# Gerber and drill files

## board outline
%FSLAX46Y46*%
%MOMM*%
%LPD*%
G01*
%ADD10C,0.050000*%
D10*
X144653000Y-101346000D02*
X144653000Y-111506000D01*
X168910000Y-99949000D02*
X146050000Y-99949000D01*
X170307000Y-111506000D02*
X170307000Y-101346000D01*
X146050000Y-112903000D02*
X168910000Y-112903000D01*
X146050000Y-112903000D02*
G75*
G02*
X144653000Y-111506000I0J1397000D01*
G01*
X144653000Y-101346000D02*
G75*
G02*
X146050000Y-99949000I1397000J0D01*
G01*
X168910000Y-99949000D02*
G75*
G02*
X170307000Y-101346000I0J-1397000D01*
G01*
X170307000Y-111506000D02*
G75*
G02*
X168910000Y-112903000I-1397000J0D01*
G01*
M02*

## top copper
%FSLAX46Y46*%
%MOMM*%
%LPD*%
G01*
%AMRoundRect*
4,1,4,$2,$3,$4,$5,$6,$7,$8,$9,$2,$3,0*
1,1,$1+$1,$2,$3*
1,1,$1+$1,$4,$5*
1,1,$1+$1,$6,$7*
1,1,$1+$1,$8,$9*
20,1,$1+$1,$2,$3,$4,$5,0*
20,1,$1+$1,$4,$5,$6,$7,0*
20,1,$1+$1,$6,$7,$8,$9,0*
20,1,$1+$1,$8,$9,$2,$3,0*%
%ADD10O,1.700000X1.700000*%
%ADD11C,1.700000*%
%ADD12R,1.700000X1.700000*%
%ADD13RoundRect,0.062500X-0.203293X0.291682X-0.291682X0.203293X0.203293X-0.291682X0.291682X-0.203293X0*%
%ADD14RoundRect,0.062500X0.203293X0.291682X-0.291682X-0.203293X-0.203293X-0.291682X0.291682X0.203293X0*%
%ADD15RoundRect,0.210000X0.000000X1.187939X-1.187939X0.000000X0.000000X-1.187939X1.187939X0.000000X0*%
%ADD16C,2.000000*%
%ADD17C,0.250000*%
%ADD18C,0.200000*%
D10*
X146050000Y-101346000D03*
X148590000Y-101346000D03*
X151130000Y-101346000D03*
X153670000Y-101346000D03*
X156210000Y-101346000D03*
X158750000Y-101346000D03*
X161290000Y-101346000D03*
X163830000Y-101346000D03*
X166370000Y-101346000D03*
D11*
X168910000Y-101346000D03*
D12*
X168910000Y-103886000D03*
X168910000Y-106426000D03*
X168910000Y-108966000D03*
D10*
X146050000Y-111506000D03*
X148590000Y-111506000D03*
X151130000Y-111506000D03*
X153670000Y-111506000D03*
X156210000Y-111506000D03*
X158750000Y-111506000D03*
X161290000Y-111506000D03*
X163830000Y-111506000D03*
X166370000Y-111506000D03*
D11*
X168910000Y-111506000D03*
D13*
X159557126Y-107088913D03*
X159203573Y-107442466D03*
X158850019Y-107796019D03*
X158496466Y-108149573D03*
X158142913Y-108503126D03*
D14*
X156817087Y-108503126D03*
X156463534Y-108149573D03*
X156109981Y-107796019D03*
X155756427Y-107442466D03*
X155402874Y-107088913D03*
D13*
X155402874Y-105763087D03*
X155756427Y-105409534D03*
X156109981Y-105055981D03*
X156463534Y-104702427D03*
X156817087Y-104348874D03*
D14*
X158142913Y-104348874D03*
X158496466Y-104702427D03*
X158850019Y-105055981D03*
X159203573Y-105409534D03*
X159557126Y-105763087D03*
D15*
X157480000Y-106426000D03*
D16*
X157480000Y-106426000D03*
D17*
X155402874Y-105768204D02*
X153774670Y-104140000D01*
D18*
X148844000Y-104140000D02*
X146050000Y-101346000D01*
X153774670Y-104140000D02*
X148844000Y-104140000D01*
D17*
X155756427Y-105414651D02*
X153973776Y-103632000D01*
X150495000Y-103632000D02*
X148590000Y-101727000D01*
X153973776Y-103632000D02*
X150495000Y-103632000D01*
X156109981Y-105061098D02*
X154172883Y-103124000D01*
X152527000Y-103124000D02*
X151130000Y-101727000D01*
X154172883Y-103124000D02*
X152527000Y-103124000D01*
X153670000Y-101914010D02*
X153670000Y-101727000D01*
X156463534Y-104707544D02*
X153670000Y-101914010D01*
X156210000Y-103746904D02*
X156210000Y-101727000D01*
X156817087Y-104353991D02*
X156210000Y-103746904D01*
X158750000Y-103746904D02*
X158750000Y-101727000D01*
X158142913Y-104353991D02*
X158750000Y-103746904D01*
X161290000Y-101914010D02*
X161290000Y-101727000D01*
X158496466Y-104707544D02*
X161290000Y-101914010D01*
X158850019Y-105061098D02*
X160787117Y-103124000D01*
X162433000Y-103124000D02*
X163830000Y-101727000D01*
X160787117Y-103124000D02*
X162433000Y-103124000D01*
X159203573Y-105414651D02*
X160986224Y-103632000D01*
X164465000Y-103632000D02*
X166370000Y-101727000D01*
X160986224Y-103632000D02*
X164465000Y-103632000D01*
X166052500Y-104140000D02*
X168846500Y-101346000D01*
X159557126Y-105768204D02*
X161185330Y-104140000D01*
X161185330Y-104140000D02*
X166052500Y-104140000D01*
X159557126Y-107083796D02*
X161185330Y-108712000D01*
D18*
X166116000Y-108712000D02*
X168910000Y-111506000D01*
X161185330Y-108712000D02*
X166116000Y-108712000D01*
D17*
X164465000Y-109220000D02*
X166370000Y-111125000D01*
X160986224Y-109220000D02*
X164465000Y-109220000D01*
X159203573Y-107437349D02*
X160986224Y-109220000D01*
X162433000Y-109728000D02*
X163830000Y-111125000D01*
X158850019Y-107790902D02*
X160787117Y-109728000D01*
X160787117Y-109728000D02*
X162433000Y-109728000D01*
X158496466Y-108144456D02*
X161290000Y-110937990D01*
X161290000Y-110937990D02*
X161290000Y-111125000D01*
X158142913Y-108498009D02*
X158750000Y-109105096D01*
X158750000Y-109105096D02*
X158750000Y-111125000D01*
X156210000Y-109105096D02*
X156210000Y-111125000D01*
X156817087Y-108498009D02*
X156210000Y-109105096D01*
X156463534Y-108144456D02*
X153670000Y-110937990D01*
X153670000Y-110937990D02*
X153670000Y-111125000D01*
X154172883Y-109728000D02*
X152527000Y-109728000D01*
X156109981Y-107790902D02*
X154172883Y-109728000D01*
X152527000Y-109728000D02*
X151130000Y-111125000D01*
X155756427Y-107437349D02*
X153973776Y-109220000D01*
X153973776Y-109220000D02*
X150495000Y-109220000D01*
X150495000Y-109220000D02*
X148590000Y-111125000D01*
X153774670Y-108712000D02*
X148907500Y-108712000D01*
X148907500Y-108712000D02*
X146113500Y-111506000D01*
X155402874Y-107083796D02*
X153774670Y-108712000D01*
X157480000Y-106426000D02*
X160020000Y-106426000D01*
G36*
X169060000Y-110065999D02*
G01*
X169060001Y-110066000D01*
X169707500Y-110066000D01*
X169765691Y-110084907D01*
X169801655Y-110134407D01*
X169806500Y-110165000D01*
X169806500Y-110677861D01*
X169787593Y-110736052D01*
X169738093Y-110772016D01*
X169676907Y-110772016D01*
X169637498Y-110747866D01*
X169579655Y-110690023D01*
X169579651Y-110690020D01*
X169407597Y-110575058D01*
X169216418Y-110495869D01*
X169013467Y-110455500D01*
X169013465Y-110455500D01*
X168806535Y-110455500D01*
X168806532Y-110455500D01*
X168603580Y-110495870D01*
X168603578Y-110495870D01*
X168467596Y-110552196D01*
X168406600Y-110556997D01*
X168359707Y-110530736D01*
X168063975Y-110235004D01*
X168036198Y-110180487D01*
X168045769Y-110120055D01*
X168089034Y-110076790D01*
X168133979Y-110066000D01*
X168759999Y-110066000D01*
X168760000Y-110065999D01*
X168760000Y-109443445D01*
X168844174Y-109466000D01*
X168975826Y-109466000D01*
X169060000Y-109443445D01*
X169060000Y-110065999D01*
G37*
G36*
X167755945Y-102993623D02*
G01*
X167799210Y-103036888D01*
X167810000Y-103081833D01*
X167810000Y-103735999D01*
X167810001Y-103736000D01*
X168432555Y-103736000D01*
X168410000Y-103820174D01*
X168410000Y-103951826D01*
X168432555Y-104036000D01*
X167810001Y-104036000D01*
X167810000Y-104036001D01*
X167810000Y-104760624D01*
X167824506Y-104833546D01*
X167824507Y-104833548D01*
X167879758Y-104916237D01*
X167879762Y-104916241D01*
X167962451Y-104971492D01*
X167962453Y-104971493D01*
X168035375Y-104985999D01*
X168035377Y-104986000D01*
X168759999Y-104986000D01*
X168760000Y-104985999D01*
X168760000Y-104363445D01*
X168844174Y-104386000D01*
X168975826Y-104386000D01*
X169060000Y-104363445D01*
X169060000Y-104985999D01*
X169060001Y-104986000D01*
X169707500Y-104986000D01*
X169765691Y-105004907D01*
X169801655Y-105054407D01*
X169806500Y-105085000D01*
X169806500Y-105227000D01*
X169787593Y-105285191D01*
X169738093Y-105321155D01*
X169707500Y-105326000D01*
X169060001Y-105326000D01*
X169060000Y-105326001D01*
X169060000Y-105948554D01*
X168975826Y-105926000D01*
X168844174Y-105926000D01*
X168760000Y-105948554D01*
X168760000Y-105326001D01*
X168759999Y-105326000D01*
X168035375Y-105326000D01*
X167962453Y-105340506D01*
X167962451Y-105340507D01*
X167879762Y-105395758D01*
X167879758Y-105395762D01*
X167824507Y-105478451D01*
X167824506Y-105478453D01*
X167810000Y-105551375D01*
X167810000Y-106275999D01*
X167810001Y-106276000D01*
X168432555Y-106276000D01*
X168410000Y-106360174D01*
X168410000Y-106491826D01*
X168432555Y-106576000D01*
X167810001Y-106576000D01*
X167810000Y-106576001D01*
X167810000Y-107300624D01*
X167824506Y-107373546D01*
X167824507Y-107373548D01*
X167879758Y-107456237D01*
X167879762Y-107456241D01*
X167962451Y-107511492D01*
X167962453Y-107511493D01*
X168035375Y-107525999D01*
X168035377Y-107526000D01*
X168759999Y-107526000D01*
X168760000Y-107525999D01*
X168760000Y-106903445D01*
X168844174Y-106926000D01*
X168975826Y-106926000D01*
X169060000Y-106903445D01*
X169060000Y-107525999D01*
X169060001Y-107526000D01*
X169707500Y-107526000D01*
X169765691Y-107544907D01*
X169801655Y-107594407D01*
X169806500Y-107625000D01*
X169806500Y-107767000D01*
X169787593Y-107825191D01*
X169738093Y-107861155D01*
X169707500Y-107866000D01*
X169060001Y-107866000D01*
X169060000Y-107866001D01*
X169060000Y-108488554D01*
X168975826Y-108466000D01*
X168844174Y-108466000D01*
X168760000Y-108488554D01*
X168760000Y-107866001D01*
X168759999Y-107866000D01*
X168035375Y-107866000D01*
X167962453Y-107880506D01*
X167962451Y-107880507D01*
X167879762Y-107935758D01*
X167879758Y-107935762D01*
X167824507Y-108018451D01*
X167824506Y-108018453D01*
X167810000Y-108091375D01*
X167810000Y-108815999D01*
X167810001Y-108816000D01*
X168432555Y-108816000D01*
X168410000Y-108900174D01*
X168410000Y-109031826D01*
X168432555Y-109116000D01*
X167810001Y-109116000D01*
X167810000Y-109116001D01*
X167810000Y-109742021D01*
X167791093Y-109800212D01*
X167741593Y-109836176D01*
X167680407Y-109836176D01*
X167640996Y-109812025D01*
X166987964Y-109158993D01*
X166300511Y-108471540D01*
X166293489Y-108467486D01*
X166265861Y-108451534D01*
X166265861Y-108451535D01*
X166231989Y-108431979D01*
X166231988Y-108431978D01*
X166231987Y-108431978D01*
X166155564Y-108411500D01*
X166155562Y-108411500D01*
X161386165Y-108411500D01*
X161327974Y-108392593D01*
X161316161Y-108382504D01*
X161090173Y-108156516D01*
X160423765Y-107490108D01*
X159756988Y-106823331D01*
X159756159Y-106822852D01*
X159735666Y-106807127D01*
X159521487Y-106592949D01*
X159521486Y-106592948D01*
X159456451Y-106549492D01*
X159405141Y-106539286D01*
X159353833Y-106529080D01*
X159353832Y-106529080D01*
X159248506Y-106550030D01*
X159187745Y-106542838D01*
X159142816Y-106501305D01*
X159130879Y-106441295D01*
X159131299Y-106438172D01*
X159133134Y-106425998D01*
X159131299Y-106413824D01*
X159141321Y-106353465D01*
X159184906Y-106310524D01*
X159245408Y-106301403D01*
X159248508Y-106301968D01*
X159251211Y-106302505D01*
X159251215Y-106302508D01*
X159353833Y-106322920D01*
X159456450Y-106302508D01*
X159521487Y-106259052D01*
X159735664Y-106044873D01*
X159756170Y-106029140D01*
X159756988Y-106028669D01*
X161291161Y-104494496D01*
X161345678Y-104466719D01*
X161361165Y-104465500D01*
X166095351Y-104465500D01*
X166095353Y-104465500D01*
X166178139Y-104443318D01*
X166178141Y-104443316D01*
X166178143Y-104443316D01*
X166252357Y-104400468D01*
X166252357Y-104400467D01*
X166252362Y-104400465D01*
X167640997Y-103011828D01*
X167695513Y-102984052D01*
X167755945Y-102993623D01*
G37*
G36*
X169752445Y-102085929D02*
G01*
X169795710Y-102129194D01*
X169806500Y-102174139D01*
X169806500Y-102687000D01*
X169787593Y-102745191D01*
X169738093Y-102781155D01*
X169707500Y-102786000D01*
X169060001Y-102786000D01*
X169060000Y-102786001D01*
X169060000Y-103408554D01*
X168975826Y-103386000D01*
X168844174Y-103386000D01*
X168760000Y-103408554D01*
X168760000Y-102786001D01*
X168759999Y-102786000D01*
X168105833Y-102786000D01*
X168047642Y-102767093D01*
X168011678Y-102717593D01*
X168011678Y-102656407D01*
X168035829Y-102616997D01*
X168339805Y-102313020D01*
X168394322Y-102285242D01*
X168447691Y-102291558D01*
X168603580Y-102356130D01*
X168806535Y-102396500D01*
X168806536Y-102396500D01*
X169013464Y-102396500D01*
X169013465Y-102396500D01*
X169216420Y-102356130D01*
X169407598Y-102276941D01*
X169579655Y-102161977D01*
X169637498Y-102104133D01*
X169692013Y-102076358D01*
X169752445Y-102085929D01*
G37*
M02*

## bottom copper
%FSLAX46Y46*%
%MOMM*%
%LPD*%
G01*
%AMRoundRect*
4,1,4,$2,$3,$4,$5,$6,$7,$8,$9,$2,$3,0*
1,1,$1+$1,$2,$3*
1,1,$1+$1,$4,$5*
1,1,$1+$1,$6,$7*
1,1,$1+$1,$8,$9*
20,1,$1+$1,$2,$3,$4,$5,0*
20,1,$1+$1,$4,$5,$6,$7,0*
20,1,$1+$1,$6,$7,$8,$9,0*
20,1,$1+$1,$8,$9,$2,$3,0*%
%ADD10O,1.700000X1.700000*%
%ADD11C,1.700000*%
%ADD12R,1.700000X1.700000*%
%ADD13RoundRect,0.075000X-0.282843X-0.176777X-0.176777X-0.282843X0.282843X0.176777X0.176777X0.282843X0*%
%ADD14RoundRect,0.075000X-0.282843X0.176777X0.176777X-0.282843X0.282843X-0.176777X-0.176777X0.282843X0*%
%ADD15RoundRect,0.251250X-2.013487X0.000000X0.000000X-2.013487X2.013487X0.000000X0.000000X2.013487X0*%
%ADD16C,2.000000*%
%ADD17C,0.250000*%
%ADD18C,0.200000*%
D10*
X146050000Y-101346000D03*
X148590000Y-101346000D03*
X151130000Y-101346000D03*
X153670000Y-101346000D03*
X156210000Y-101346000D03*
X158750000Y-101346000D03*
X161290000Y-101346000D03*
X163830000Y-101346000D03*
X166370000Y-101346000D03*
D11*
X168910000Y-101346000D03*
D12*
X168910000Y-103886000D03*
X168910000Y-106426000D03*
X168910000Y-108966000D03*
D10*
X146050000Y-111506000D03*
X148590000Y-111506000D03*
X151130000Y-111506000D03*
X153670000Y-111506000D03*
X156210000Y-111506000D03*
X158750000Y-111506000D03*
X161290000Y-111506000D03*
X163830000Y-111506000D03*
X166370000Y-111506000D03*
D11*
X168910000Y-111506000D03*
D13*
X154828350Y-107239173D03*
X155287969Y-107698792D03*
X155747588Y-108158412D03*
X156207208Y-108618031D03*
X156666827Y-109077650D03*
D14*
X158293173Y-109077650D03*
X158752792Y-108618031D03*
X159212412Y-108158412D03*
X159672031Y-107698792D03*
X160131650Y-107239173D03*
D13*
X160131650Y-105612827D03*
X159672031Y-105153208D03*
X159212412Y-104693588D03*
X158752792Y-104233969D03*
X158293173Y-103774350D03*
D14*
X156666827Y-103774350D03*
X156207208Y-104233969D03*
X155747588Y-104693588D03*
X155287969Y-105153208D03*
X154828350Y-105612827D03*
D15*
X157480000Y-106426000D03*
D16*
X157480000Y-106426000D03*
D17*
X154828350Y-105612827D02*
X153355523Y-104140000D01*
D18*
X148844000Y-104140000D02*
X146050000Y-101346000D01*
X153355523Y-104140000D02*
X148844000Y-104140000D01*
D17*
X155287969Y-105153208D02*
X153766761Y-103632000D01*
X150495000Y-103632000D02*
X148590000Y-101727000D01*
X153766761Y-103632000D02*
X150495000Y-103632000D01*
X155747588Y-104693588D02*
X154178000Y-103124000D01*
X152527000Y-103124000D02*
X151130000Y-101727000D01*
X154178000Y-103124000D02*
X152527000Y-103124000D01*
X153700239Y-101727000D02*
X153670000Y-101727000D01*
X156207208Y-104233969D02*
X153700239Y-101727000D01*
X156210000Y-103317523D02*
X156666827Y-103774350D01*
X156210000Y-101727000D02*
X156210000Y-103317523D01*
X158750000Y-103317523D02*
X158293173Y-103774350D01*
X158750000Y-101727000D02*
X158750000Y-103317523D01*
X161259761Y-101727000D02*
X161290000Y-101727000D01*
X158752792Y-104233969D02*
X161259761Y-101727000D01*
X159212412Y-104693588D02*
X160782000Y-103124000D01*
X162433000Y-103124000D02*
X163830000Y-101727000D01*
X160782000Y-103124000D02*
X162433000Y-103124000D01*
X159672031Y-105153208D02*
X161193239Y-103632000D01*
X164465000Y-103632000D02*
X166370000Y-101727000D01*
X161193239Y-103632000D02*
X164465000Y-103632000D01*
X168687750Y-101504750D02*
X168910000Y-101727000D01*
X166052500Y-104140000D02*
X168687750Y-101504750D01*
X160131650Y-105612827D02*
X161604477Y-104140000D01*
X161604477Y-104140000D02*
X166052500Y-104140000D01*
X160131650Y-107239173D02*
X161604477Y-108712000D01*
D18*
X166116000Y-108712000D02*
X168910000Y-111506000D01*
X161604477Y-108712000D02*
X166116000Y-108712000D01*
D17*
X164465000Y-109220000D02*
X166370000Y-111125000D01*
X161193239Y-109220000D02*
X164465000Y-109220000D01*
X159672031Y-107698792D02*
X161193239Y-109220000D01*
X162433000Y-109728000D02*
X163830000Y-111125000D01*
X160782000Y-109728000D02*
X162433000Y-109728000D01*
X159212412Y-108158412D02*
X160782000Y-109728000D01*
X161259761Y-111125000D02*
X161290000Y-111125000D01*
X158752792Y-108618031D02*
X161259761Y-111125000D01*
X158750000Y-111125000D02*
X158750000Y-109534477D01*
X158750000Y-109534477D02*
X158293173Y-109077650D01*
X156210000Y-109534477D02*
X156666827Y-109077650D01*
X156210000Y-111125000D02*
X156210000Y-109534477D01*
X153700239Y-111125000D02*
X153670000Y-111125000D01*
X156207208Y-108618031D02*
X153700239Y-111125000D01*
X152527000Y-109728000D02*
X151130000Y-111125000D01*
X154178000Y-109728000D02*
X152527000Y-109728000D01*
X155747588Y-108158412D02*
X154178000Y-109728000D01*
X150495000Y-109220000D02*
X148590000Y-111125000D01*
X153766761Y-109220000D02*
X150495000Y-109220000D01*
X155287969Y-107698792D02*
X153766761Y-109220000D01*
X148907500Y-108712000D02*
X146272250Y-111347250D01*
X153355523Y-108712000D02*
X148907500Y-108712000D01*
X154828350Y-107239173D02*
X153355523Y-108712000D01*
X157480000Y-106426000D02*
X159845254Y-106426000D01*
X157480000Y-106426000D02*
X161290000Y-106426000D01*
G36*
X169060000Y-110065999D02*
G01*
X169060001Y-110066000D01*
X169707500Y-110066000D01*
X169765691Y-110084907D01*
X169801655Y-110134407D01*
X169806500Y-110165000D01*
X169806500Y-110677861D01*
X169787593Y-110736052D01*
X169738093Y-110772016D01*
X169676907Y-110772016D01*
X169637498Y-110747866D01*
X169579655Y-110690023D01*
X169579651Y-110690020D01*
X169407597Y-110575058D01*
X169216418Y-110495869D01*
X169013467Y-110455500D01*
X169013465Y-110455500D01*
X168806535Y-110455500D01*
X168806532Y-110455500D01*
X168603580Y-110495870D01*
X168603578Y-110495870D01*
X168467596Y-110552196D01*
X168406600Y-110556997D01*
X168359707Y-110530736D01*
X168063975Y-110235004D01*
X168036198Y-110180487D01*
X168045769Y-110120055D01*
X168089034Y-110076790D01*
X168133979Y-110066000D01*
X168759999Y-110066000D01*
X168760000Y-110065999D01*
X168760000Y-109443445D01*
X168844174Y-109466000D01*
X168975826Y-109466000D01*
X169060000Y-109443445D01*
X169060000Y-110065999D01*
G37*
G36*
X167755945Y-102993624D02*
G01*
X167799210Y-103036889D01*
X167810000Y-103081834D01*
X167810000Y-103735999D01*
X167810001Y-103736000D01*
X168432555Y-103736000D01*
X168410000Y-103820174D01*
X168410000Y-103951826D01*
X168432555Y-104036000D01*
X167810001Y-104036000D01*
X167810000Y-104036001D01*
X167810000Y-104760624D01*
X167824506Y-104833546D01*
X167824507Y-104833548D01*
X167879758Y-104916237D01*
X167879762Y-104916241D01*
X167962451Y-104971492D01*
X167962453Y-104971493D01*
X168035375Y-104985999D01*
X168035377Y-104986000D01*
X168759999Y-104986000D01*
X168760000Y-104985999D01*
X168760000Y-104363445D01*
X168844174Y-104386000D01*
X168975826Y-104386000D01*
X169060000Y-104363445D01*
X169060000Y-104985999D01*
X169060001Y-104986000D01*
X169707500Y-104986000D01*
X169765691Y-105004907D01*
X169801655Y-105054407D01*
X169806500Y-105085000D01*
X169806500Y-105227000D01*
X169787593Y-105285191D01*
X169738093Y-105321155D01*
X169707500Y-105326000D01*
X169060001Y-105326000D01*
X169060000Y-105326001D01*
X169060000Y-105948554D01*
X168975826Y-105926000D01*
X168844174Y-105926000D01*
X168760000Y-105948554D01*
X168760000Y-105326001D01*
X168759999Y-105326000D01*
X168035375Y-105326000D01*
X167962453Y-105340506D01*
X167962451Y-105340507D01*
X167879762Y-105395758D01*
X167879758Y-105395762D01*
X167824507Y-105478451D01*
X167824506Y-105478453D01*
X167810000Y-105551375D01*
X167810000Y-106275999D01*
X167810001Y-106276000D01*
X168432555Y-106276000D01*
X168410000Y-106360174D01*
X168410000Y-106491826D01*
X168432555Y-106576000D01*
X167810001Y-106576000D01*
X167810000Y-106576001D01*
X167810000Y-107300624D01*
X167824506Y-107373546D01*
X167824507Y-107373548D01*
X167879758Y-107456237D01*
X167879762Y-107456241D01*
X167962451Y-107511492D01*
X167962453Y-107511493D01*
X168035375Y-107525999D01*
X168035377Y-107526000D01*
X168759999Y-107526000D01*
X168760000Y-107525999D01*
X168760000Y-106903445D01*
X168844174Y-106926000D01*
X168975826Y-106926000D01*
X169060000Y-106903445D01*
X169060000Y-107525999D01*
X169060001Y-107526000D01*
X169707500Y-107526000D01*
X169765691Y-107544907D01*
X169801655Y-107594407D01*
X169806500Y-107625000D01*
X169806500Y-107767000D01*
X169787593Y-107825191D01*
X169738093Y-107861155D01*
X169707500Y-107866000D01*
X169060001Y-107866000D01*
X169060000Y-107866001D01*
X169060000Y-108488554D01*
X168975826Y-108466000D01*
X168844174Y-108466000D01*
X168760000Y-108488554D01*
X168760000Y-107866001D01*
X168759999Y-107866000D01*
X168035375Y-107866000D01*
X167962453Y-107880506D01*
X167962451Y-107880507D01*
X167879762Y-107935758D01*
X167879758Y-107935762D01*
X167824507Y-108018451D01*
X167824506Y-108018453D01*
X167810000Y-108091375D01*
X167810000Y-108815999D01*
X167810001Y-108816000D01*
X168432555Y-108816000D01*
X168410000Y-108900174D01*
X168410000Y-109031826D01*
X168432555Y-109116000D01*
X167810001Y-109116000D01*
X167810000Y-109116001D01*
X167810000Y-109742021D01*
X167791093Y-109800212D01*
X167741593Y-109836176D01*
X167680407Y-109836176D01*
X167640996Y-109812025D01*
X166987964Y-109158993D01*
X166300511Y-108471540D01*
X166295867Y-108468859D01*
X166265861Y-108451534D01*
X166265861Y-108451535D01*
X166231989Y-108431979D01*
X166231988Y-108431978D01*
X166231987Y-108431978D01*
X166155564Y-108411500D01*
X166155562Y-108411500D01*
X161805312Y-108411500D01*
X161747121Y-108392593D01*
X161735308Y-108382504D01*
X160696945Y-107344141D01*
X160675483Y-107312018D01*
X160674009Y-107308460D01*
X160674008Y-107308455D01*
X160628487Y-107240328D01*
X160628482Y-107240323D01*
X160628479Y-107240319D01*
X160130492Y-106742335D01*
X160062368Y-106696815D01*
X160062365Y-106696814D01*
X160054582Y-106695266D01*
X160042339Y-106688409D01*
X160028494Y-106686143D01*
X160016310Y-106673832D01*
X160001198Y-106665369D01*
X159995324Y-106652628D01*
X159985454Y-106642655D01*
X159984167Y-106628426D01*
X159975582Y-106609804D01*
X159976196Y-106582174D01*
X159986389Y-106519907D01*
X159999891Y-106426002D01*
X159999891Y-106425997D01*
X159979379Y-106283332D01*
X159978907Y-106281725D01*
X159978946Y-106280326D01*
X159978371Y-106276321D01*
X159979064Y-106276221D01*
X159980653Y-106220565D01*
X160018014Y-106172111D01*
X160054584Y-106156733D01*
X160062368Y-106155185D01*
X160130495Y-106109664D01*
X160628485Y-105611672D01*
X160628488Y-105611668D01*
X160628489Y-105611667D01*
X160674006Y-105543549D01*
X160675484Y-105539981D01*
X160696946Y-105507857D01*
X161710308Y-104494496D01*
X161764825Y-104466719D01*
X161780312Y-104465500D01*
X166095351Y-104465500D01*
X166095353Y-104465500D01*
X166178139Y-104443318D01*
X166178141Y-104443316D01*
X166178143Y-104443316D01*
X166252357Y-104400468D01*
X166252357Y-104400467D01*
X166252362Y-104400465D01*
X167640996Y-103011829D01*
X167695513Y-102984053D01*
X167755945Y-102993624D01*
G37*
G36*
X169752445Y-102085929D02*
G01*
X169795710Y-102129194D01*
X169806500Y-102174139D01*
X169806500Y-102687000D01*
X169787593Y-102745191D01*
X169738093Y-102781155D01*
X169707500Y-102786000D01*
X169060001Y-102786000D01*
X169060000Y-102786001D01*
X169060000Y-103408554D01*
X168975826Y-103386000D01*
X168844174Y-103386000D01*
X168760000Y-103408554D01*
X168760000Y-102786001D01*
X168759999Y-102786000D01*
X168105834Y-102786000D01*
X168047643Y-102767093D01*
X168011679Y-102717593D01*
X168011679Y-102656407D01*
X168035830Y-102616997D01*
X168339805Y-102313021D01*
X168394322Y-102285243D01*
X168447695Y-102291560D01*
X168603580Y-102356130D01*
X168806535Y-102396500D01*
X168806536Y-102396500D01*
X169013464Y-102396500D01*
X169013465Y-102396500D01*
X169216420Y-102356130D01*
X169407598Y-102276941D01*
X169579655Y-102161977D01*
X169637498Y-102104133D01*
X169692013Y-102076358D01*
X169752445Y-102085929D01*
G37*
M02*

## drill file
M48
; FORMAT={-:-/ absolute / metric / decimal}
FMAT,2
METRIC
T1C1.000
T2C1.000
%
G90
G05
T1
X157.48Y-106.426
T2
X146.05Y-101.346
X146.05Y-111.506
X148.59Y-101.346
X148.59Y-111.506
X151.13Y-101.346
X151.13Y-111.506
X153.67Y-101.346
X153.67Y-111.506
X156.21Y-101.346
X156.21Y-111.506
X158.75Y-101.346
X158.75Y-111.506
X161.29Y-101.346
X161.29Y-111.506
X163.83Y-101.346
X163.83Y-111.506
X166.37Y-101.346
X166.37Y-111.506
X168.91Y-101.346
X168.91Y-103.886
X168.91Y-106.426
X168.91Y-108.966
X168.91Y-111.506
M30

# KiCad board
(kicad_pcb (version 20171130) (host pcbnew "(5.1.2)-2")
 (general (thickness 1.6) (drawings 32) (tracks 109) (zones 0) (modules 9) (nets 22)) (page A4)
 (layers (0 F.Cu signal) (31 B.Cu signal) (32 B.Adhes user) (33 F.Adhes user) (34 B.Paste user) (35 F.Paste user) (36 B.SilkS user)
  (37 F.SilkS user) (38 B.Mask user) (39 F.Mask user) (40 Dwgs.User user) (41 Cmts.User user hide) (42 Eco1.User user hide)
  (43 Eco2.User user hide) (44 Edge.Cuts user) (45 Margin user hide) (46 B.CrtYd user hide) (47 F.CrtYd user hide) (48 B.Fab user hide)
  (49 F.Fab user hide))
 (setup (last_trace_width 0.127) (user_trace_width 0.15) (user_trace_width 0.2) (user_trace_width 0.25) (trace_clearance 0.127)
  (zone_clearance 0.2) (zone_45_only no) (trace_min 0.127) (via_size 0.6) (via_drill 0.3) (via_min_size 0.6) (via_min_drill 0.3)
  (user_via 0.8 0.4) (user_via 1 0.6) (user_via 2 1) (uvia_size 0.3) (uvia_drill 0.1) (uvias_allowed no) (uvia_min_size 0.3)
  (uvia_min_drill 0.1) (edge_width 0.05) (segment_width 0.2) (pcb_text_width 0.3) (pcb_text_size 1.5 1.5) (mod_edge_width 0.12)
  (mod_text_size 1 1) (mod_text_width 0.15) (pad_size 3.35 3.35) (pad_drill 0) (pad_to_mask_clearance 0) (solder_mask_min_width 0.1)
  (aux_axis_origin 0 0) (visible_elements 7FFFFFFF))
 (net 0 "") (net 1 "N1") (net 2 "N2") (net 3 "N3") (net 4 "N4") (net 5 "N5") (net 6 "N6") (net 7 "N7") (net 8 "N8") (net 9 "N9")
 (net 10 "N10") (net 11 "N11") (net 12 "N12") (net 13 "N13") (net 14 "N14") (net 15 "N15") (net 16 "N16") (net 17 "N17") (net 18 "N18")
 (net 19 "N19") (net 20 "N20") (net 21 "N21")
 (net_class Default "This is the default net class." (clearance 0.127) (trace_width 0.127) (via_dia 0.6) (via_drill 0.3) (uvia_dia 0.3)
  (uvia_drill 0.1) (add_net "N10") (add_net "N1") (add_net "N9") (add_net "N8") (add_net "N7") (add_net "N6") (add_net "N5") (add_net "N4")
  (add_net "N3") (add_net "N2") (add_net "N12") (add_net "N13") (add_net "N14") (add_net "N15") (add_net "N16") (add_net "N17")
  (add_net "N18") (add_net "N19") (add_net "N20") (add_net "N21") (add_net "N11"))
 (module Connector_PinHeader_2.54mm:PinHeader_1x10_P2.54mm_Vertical (layer F.Cu) (at 168.91 101.346 270)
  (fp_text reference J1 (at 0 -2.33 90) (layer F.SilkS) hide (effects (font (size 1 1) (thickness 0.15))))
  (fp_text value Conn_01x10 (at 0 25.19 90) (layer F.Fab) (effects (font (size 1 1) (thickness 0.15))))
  (pad 10 thru_hole oval (at 0 22.86 270) (size 1.7 1.7) (drill 1) (layers *.Cu *.Mask) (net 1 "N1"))
  (pad 9 thru_hole oval (at 0 20.32 270) (size 1.7 1.7) (drill 1) (layers *.Cu *.Mask) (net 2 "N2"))
  (pad 8 thru_hole oval (at 0 17.78 270) (size 1.7 1.7) (drill 1) (layers *.Cu *.Mask) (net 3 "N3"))
  (pad 7 thru_hole oval (at 0 15.24 270) (size 1.7 1.7) (drill 1) (layers *.Cu *.Mask) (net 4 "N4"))
  (pad 6 thru_hole oval (at 0 12.7 270) (size 1.7 1.7) (drill 1) (layers *.Cu *.Mask) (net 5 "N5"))
  (pad 5 thru_hole oval (at 0 10.16 270) (size 1.7 1.7) (drill 1) (layers *.Cu *.Mask) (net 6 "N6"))
  (pad 4 thru_hole oval (at 0 7.62 270) (size 1.7 1.7) (drill 1) (layers *.Cu *.Mask) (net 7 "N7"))
  (pad 3 thru_hole oval (at 0 5.08 270) (size 1.7 1.7) (drill 1) (layers *.Cu *.Mask) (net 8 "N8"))
  (pad 2 thru_hole oval (at 0 2.54 270) (size 1.7 1.7) (drill 1) (layers *.Cu *.Mask) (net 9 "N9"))
  (pad 1 thru_hole circle (at 0 0 270) (size 1.7 1.7) (drill 1) (layers *.Cu *.Mask) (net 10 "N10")))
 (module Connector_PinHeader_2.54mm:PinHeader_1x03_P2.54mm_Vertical (layer B.Cu) (at 168.91 103.886 180)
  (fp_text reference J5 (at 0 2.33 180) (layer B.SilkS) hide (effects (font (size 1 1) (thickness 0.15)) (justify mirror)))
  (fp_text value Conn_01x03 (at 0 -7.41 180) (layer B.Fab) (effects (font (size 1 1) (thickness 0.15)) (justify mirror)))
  (pad 1 thru_hole rect (at 0 0 180) (size 1.7 1.7) (drill 1) (layers *.Cu *.Mask) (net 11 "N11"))
  (pad 2 thru_hole rect (at 0 -2.54 180) (size 1.7 1.7) (drill 1) (layers *.Cu *.Mask) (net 11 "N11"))
  (pad 3 thru_hole rect (at 0 -5.08 180) (size 1.7 1.7) (drill 1) (layers *.Cu *.Mask) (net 11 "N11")))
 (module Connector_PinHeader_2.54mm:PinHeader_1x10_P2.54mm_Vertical (layer F.Cu) (at 168.91 111.506 270)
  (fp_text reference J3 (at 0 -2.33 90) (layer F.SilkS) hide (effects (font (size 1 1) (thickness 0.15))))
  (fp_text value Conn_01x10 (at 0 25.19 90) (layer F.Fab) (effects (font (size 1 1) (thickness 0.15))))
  (pad 10 thru_hole oval (at 0 22.86 270) (size 1.7 1.7) (drill 1) (layers *.Cu *.Mask) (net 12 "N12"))
  (pad 9 thru_hole oval (at 0 20.32 270) (size 1.7 1.7) (drill 1) (layers *.Cu *.Mask) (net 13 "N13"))
  (pad 8 thru_hole oval (at 0 17.78 270) (size 1.7 1.7) (drill 1) (layers *.Cu *.Mask) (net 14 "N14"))
  (pad 7 thru_hole oval (at 0 15.24 270) (size 1.7 1.7) (drill 1) (layers *.Cu *.Mask) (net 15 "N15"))
  (pad 6 thru_hole oval (at 0 12.7 270) (size 1.7 1.7) (drill 1) (layers *.Cu *.Mask) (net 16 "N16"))
  (pad 5 thru_hole oval (at 0 10.16 270) (size 1.7 1.7) (drill 1) (layers *.Cu *.Mask) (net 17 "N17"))
  (pad 4 thru_hole oval (at 0 7.62 270) (size 1.7 1.7) (drill 1) (layers *.Cu *.Mask) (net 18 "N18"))
  (pad 3 thru_hole oval (at 0 5.08 270) (size 1.7 1.7) (drill 1) (layers *.Cu *.Mask) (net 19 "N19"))
  (pad 2 thru_hole oval (at 0 2.54 270) (size 1.7 1.7) (drill 1) (layers *.Cu *.Mask) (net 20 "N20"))
  (pad 1 thru_hole circle (at 0 0 270) (size 1.7 1.7) (drill 1) (layers *.Cu *.Mask) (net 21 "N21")))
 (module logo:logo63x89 (layer B.Cu) (at 148.209 106.299 270)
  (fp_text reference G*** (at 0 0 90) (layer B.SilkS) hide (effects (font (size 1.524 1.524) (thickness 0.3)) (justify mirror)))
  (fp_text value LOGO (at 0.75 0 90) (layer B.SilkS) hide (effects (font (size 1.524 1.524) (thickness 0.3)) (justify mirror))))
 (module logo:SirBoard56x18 (layer B.Cu) (at 152.654 106.426 270)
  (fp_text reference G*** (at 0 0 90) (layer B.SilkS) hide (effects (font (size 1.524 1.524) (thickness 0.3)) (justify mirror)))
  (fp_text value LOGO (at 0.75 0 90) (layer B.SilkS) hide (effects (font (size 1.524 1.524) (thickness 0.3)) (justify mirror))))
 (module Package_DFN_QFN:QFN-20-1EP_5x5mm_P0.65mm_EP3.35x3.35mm (layer B.Cu) (at 157.48 106.426 315)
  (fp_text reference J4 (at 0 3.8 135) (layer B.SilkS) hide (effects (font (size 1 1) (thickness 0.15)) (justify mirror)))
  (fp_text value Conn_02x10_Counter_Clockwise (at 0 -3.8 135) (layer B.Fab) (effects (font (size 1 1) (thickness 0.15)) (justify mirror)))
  (pad 20 smd roundrect (at -1.3 2.45 315) (size 0.3 0.8) (layers B.Cu B.Paste B.Mask) (roundrect_rratio 0.25) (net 12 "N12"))
  (pad 19 smd roundrect (at -0.65 2.45 315) (size 0.3 0.8) (layers B.Cu B.Paste B.Mask) (roundrect_rratio 0.25) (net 13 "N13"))
  (pad 18 smd roundrect (at 0 2.45 315) (size 0.3 0.8) (layers B.Cu B.Paste B.Mask) (roundrect_rratio 0.25) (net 14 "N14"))
  (pad 17 smd roundrect (at 0.65 2.45 315) (size 0.3 0.8) (layers B.Cu B.Paste B.Mask) (roundrect_rratio 0.25) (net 15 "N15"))
  (pad 16 smd roundrect (at 1.3 2.45 315) (size 0.3 0.8) (layers B.Cu B.Paste B.Mask) (roundrect_rratio 0.25) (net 16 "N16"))
  (pad 15 smd roundrect (at 2.45 1.3 315) (size 0.8 0.3) (layers B.Cu B.Paste B.Mask) (roundrect_rratio 0.25) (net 17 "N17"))
  (pad 14 smd roundrect (at 2.45 0.65 315) (size 0.8 0.3) (layers B.Cu B.Paste B.Mask) (roundrect_rratio 0.25) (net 18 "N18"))
  (pad 13 smd roundrect (at 2.45 0 315) (size 0.8 0.3) (layers B.Cu B.Paste B.Mask) (roundrect_rratio 0.25) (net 19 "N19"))
  (pad 12 smd roundrect (at 2.45 -0.65 315) (size 0.8 0.3) (layers B.Cu B.Paste B.Mask) (roundrect_rratio 0.25) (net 20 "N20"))
  (pad 11 smd roundrect (at 2.45 -1.3 315) (size 0.8 0.3) (layers B.Cu B.Paste B.Mask) (roundrect_rratio 0.25) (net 21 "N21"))
  (pad 10 smd roundrect (at 1.3 -2.45 315) (size 0.3 0.8) (layers B.Cu B.Paste B.Mask) (roundrect_rratio 0.25) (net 10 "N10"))
  (pad 9 smd roundrect (at 0.65 -2.45 315) (size 0.3 0.8) (layers B.Cu B.Paste B.Mask) (roundrect_rratio 0.25) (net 9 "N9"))
  (pad 8 smd roundrect (at 0 -2.45 315) (size 0.3 0.8) (layers B.Cu B.Paste B.Mask) (roundrect_rratio 0.25) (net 8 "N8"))
  (pad 7 smd roundrect (at -0.65 -2.45 315) (size 0.3 0.8) (layers B.Cu B.Paste B.Mask) (roundrect_rratio 0.25) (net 7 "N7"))
  (pad 6 smd roundrect (at -1.3 -2.45 315) (size 0.3 0.8) (layers B.Cu B.Paste B.Mask) (roundrect_rratio 0.25) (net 6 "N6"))
  (pad 5 smd roundrect (at -2.45 -1.3 315) (size 0.8 0.3) (layers B.Cu B.Paste B.Mask) (roundrect_rratio 0.25) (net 5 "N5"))
  (pad 4 smd roundrect (at -2.45 -0.65 315) (size 0.8 0.3) (layers B.Cu B.Paste B.Mask) (roundrect_rratio 0.25) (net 4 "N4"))
  (pad 3 smd roundrect (at -2.45 0 315) (size 0.8 0.3) (layers B.Cu B.Paste B.Mask) (roundrect_rratio 0.25) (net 3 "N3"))
  (pad 2 smd roundrect (at -2.45 0.65 315) (size 0.8 0.3) (layers B.Cu B.Paste B.Mask) (roundrect_rratio 0.25) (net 2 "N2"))
  (pad 1 smd roundrect (at -2.45 1.3 315) (size 0.8 0.3) (layers B.Cu B.Paste B.Mask) (roundrect_rratio 0.25) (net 1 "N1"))
  (pad "" smd roundrect (at 0.84 -0.84 315) (size 1.35 1.35) (layers B.Paste) (roundrect_rratio 0.185185))
  (pad "" smd roundrect (at 0.84 0.84 315) (size 1.35 1.35) (layers B.Paste) (roundrect_rratio 0.185185))
  (pad "" smd roundrect (at -0.84 -0.84 315) (size 1.35 1.35) (layers B.Paste) (roundrect_rratio 0.185185))
  (pad "" smd roundrect (at -0.84 0.84 315) (size 1.35 1.35) (layers B.Paste) (roundrect_rratio 0.185185))
  (pad 21 smd roundrect (at 0 0 315) (size 3.35 3.35) (layers B.Cu B.Mask) (roundrect_rratio 0.075) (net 11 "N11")))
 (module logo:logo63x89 (layer F.Cu) (at 148.336 106.426 90)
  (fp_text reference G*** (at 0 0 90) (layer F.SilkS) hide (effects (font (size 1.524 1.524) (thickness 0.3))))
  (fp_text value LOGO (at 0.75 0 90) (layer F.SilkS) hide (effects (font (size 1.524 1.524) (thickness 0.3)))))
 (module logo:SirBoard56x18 (layer F.Cu) (at 152.654 106.426 90)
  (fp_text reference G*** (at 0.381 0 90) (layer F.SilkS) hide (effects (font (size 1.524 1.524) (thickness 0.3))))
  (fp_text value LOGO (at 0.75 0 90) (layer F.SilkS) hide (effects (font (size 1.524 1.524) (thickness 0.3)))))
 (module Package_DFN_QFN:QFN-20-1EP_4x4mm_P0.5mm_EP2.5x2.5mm (layer F.Cu) (at 157.48 106.426 225)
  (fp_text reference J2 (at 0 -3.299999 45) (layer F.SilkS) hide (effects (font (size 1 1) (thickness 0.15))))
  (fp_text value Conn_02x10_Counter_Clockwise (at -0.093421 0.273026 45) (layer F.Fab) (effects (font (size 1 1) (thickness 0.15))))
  (pad 20 smd roundrect (at -1 -1.9375 225) (size 0.25 0.825) (layers F.Cu F.Paste F.Mask) (roundrect_rratio 0.25) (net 21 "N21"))
  (pad 19 smd roundrect (at -0.5 -1.9375 225) (size 0.25 0.825) (layers F.Cu F.Paste F.Mask) (roundrect_rratio 0.25) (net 20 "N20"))
  (pad 18 smd roundrect (at 0 -1.9375 225) (size 0.25 0.825) (layers F.Cu F.Paste F.Mask) (roundrect_rratio 0.25) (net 19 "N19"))
  (pad 17 smd roundrect (at 0.5 -1.9375 225) (size 0.25 0.825) (layers F.Cu F.Paste F.Mask) (roundrect_rratio 0.25) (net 18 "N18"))
  (pad 16 smd roundrect (at 1 -1.9375 225) (size 0.25 0.825) (layers F.Cu F.Paste F.Mask) (roundrect_rratio 0.25) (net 17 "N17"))
  (pad 15 smd roundrect (at 1.9375 -1 225) (size 0.825 0.25) (layers F.Cu F.Paste F.Mask) (roundrect_rratio 0.25) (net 16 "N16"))
  (pad 14 smd roundrect (at 1.9375 -0.5 225) (size 0.825 0.25) (layers F.Cu F.Paste F.Mask) (roundrect_rratio 0.25) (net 15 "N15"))
  (pad 13 smd roundrect (at 1.9375 0 225) (size 0.825 0.25) (layers F.Cu F.Paste F.Mask) (roundrect_rratio 0.25) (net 14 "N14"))
  (pad 12 smd roundrect (at 1.9375 0.5 225) (size 0.825 0.25) (layers F.Cu F.Paste F.Mask) (roundrect_rratio 0.25) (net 13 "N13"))
  (pad 11 smd roundrect (at 1.9375 1 225) (size 0.825 0.25) (layers F.Cu F.Paste F.Mask) (roundrect_rratio 0.25) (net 12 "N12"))
  (pad 10 smd roundrect (at 1 1.9375 225) (size 0.25 0.825) (layers F.Cu F.Paste F.Mask) (roundrect_rratio 0.25) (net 1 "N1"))
  (pad 9 smd roundrect (at 0.5 1.9375 225) (size 0.25 0.825) (layers F.Cu F.Paste F.Mask) (roundrect_rratio 0.25) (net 2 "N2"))
  (pad 8 smd roundrect (at 0 1.9375 225) (size 0.25 0.825) (layers F.Cu F.Paste F.Mask) (roundrect_rratio 0.25) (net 3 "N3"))
  (pad 7 smd roundrect (at -0.5 1.9375 225) (size 0.25 0.825) (layers F.Cu F.Paste F.Mask) (roundrect_rratio 0.25) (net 4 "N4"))
  (pad 6 smd roundrect (at -1 1.9375 225) (size 0.25 0.825) (layers F.Cu F.Paste F.Mask) (roundrect_rratio 0.25) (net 5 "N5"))
  (pad 5 smd roundrect (at -1.9375 1 225) (size 0.825 0.25) (layers F.Cu F.Paste F.Mask) (roundrect_rratio 0.25) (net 6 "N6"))
  (pad 4 smd roundrect (at -1.9375 0.5 225) (size 0.825 0.25) (layers F.Cu F.Paste F.Mask) (roundrect_rratio 0.25) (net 7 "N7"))
  (pad 3 smd roundrect (at -1.9375 0 225) (size 0.825 0.25) (layers F.Cu F.Paste F.Mask) (roundrect_rratio 0.25) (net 8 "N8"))
  (pad 2 smd roundrect (at -1.9375 -0.5 225) (size 0.825 0.25) (layers F.Cu F.Paste F.Mask) (roundrect_rratio 0.25) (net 9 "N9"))
  (pad 1 smd roundrect (at -1.9375 -1 225) (size 0.825 0.25) (layers F.Cu F.Paste F.Mask) (roundrect_rratio 0.25) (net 10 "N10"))
  (pad "" smd roundrect (at 0.625 0.625 225) (size 1.01 1.01) (layers F.Paste) (roundrect_rratio 0.247525))
  (pad "" smd roundrect (at 0.625 -0.625 225) (size 1.01 1.01) (layers F.Paste) (roundrect_rratio 0.247525))
  (pad "" smd roundrect (at -0.625 0.625 225) (size 1.01 1.01) (layers F.Paste) (roundrect_rratio 0.247525))
  (pad "" smd roundrect (at -0.625 -0.625 225) (size 1.01 1.01) (layers F.Paste) (roundrect_rratio 0.247525))
  (pad 21 smd roundrect (at 0 0 225) (size 2.1 2.1) (layers F.Cu F.Mask) (roundrect_rratio 0.1) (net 11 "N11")))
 (gr_line (start 144.653 101.346) (end 144.653 111.506) (layer Edge.Cuts) (width 0.05))
 (gr_line (start 168.91 99.949) (end 146.05 99.949) (layer Edge.Cuts) (width 0.05))
 (gr_line (start 170.307 111.506) (end 170.307 101.346) (layer Edge.Cuts) (width 0.05))
 (gr_line (start 146.05 112.903) (end 168.91 112.903) (layer Edge.Cuts) (width 0.05))
 (gr_arc (start 146.05 111.506) (end 144.653 111.506) (angle -90) (layer Edge.Cuts) (width 0.05))
 (gr_arc (start 146.05 101.346) (end 146.05 99.949) (angle -90) (layer Edge.Cuts) (width 0.05))
 (gr_arc (start 168.91 101.346) (end 170.307 101.346) (angle -90) (layer Edge.Cuts) (width 0.05))
 (gr_arc (start 168.91 111.506) (end 168.91 112.903) (angle -90) (layer Edge.Cuts) (width 0.05))
 (segment (start 155.402874 105.768204) (end 153.77467 104.14) (width 0.25) (layer F.Cu) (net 1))
 (segment (start 154.82835 105.612827) (end 153.355523 104.14) (width 0.25) (layer B.Cu) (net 1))
 (segment (start 148.844 104.14) (end 146.05 101.346) (width 0.2) (layer B.Cu) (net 1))
 (segment (start 148.844 104.14) (end 146.05 101.346) (width 0.2) (layer F.Cu) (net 1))
 (segment (start 153.77467 104.14) (end 148.844 104.14) (width 0.2) (layer F.Cu) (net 1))
 (segment (start 153.355523 104.14) (end 148.844 104.14) (width 0.2) (layer B.Cu) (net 1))
 (segment (start 155.756427 105.414651) (end 153.973776 103.632) (width 0.25) (layer F.Cu) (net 2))
 (segment (start 150.495 103.632) (end 148.59 101.727) (width 0.25) (layer F.Cu) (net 2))
 (segment (start 153.973776 103.632) (end 150.495 103.632) (width 0.25) (layer F.Cu) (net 2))
 (segment (start 155.287969 105.153208) (end 153.766761 103.632) (width 0.25) (layer B.Cu) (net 2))
 (segment (start 150.495 103.632) (end 148.59 101.727) (width 0.25) (layer B.Cu) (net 2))
 (segment (start 153.766761 103.632) (end 150.495 103.632) (width 0.25) (layer B.Cu) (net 2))
 (segment (start 156.109981 105.061098) (end 154.172883 103.124) (width 0.25) (layer F.Cu) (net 3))
 (segment (start 152.527 103.124) (end 151.13 101.727) (width 0.25) (layer F.Cu) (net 3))
 (segment (start 154.172883 103.124) (end 152.527 103.124) (width 0.25) (layer F.Cu) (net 3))
 (segment (start 155.747588 104.693588) (end 154.178 103.124) (width 0.25) (layer B.Cu) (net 3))
 (segment (start 152.527 103.124) (end 151.13 101.727) (width 0.25) (layer B.Cu) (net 3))
 (segment (start 154.178 103.124) (end 152.527 103.124) (width 0.25) (layer B.Cu) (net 3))
 (segment (start 153.67 101.91401) (end 153.67 101.727) (width 0.25) (layer F.Cu) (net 4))
 (segment (start 156.463534 104.707544) (end 153.67 101.91401) (width 0.25) (layer F.Cu) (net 4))
 (segment (start 153.700239 101.727) (end 153.67 101.727) (width 0.25) (layer B.Cu) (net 4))
 (segment (start 156.207208 104.233969) (end 153.700239 101.727) (width 0.25) (layer B.Cu) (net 4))
 (segment (start 156.21 103.746904) (end 156.21 101.727) (width 0.25) (layer F.Cu) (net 5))
 (segment (start 156.817087 104.353991) (end 156.21 103.746904) (width 0.25) (layer F.Cu) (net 5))
 (segment (start 156.21 103.317523) (end 156.666827 103.77435) (width 0.25) (layer B.Cu) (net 5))
 (segment (start 156.21 101.727) (end 156.21 103.317523) (width 0.25) (layer B.Cu) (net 5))
 (segment (start 158.75 103.746904) (end 158.75 101.727) (width 0.25) (layer F.Cu) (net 6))
 (segment (start 158.142913 104.353991) (end 158.75 103.746904) (width 0.25) (layer F.Cu) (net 6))
 (segment (start 158.75 103.317523) (end 158.293173 103.77435) (width 0.25) (layer B.Cu) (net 6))
 (segment (start 158.75 101.727) (end 158.75 103.317523) (width 0.25) (layer B.Cu) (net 6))
 (segment (start 161.29 101.91401) (end 161.29 101.727) (width 0.25) (layer F.Cu) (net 7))
 (segment (start 158.496466 104.707544) (end 161.29 101.91401) (width 0.25) (layer F.Cu) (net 7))
 (segment (start 161.259761 101.727) (end 161.29 101.727) (width 0.25) (layer B.Cu) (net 7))
 (segment (start 158.752792 104.233969) (end 161.259761 101.727) (width 0.25) (layer B.Cu) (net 7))
 (segment (start 158.850019 105.061098) (end 160.787117 103.124) (width 0.25) (layer F.Cu) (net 8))
 (segment (start 162.433 103.124) (end 163.83 101.727) (width 0.25) (layer F.Cu) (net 8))
 (segment (start 160.787117 103.124) (end 162.433 103.124) (width 0.25) (layer F.Cu) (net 8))
 (segment (start 159.212412 104.693588) (end 160.782 103.124) (width 0.25) (layer B.Cu) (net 8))
 (segment (start 162.433 103.124) (end 163.83 101.727) (width 0.25) (layer B.Cu) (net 8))
 (segment (start 160.782 103.124) (end 162.433 103.124) (width 0.25) (layer B.Cu) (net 8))
 (segment (start 159.203573 105.414651) (end 160.986224 103.632) (width 0.25) (layer F.Cu) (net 9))
 (segment (start 164.465 103.632) (end 166.37 101.727) (width 0.25) (layer F.Cu) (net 9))
 (segment (start 160.986224 103.632) (end 164.465 103.632) (width 0.25) (layer F.Cu) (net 9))
 (segment (start 159.672031 105.153208) (end 161.193239 103.632) (width 0.25) (layer B.Cu) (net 9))
 (segment (start 164.465 103.632) (end 166.37 101.727) (width 0.25) (layer B.Cu) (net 9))
 (segment (start 161.193239 103.632) (end 164.465 103.632) (width 0.25) (layer B.Cu) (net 9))
 (segment (start 166.0525 104.14) (end 168.8465 101.346) (width 0.25) (layer F.Cu) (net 10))
 (segment (start 159.557126 105.768204) (end 161.18533 104.14) (width 0.25) (layer F.Cu) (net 10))
 (segment (start 161.18533 104.14) (end 166.0525 104.14) (width 0.25) (layer F.Cu) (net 10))
 (segment (start 168.68775 101.50475) (end 168.91 101.727) (width 0.25) (layer B.Cu) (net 10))
 (segment (start 166.0525 104.14) (end 168.68775 101.50475) (width 0.25) (layer B.Cu) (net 10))
 (segment (start 160.13165 105.612827) (end 161.604477 104.14) (width 0.25) (layer B.Cu) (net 10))
 (segment (start 161.604477 104.14) (end 166.0525 104.14) (width 0.25) (layer B.Cu) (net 10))
 (segment (start 160.13165 107.239173) (end 161.604477 108.712) (width 0.25) (layer B.Cu) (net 21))
 (segment (start 159.557126 107.083796) (end 161.18533 108.712) (width 0.25) (layer F.Cu) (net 21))
 (segment (start 166.116 108.712) (end 168.91 111.506) (width 0.2) (layer B.Cu) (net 21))
 (segment (start 161.604477 108.712) (end 166.116 108.712) (width 0.2) (layer B.Cu) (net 21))
 (segment (start 166.116 108.712) (end 168.91 111.506) (width 0.2) (layer F.Cu) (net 21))
 (segment (start 161.18533 108.712) (end 166.116 108.712) (width 0.2) (layer F.Cu) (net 21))
 (segment (start 164.465 109.22) (end 166.37 111.125) (width 0.25) (layer B.Cu) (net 20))
 (segment (start 161.193239 109.22) (end 164.465 109.22) (width 0.25) (layer B.Cu) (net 20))
 (segment (start 159.672031 107.698792) (end 161.193239 109.22) (width 0.25) (layer B.Cu) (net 20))
 (segment (start 164.465 109.22) (end 166.37 111.125) (width 0.25) (layer F.Cu) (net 20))
 (segment (start 160.986224 109.22) (end 164.465 109.22) (width 0.25) (layer F.Cu) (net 20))
 (segment (start 159.203573 107.437349) (end 160.986224 109.22) (width 0.25) (layer F.Cu) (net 20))
 (segment (start 162.433 109.728) (end 163.83 111.125) (width 0.25) (layer B.Cu) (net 19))
 (segment (start 160.782 109.728) (end 162.433 109.728) (width 0.25) (layer B.Cu) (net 19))
 (segment (start 159.212412 108.158412) (end 160.782 109.728) (width 0.25) (layer B.Cu) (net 19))
 (segment (start 162.433 109.728) (end 163.83 111.125) (width 0.25) (layer F.Cu) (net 19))
 (segment (start 158.850019 107.790902) (end 160.787117 109.728) (width 0.25) (layer F.Cu) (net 19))
 (segment (start 160.787117 109.728) (end 162.433 109.728) (width 0.25) (layer F.Cu) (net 19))
 (segment (start 161.259761 111.125) (end 161.29 111.125) (width 0.25) (layer B.Cu) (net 18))
 (segment (start 158.752792 108.618031) (end 161.259761 111.125) (width 0.25) (layer B.Cu) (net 18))
 (segment (start 158.496466 108.144456) (end 161.29 110.93799) (width 0.25) (layer F.Cu) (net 18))
 (segment (start 161.29 110.93799) (end 161.29 111.125) (width 0.25) (layer F.Cu) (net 18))
 (segment (start 158.75 111.125) (end 158.75 109.534477) (width 0.25) (layer B.Cu) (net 17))
 (segment (start 158.75 109.534477) (end 158.293173 109.07765) (width 0.25) (layer B.Cu) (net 17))
 (segment (start 158.142913 108.498009) (end 158.75 109.105096) (width 0.25) (layer F.Cu) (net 17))
 (segment (start 158.75 109.105096) (end 158.75 111.125) (width 0.25) (layer F.Cu) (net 17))
 (segment (start 156.21 109.534477) (end 156.666827 109.07765) (width 0.25) (layer B.Cu) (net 16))
 (segment (start 156.21 111.125) (end 156.21 109.534477) (width 0.25) (layer B.Cu) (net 16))
 (segment (start 156.21 109.105096) (end 156.21 111.125) (width 0.25) (layer F.Cu) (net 16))
 (segment (start 156.817087 108.498009) (end 156.21 109.105096) (width 0.25) (layer F.Cu) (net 16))
 (segment (start 153.700239 111.125) (end 153.67 111.125) (width 0.25) (layer B.Cu) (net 15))
 (segment (start 156.207208 108.618031) (end 153.700239 111.125) (width 0.25) (layer B.Cu) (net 15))
 (segment (start 156.463534 108.144456) (end 153.67 110.93799) (width 0.25) (layer F.Cu) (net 15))
 (segment (start 153.67 110.93799) (end 153.67 111.125) (width 0.25) (layer F.Cu) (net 15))
 (segment (start 152.527 109.728) (end 151.13 111.125) (width 0.25) (layer B.Cu) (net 14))
 (segment (start 154.178 109.728) (end 152.527 109.728) (width 0.25) (layer B.Cu) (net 14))
 (segment (start 155.747588 108.158412) (end 154.178 109.728) (width 0.25) (layer B.Cu) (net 14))
 (segment (start 154.172883 109.728) (end 152.527 109.728) (width 0.25) (layer F.Cu) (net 14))
 (segment (start 156.109981 107.790902) (end 154.172883 109.728) (width 0.25) (layer F.Cu) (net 14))
 (segment (start 152.527 109.728) (end 151.13 111.125) (width 0.25) (layer F.Cu) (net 14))
 (segment (start 150.495 109.22) (end 148.59 111.125) (width 0.25) (layer B.Cu) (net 13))
 (segment (start 153.766761 109.22) (end 150.495 109.22) (width 0.25) (layer B.Cu) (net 13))
 (segment (start 155.287969 107.698792) (end 153.766761 109.22) (width 0.25) (layer B.Cu) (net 13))
 (segment (start 155.756427 107.437349) (end 153.973776 109.22) (width 0.25) (layer F.Cu) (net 13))
 (segment (start 153.973776 109.22) (end 150.495 109.22) (width 0.25) (layer F.Cu) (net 13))
 (segment (start 150.495 109.22) (end 148.59 111.125) (width 0.25) (layer F.Cu) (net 13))
 (segment (start 153.77467 108.712) (end 148.9075 108.712) (width 0.25) (layer F.Cu) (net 12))
 (segment (start 148.9075 108.712) (end 146.1135 111.506) (width 0.25) (layer F.Cu) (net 12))
 (segment (start 148.9075 108.712) (end 146.27225 111.34725) (width 0.25) (layer B.Cu) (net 12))
 (segment (start 153.355523 108.712) (end 148.9075 108.712) (width 0.25) (layer B.Cu) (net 12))
 (segment (start 154.82835 107.239173) (end 153.355523 108.712) (width 0.25) (layer B.Cu) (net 12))
 (segment (start 155.402874 107.083796) (end 153.77467 108.712) (width 0.25) (layer F.Cu) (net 12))
 (via (at 157.48 106.426) (size 2) (drill 1) (layers F.Cu B.Cu) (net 11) (status 1000000))
 (segment (start 157.48 106.426) (end 159.845254 106.426) (width 0.25) (layer B.Cu) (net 11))
 (segment (start 157.48 106.426) (end 161.29 106.426) (width 0.25) (layer B.Cu) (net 11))
 (segment (start 157.48 106.426) (end 160.02 106.426) (width 0.25) (layer F.Cu) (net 11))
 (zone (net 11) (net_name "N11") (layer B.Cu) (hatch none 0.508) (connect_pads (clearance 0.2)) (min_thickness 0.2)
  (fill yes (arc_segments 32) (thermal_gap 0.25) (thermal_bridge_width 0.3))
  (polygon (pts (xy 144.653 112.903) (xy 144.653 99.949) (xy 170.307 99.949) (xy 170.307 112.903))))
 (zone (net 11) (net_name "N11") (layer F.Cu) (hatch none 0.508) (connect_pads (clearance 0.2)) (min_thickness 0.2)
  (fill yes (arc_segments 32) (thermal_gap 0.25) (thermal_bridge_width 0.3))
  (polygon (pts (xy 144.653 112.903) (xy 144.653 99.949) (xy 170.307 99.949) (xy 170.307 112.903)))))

